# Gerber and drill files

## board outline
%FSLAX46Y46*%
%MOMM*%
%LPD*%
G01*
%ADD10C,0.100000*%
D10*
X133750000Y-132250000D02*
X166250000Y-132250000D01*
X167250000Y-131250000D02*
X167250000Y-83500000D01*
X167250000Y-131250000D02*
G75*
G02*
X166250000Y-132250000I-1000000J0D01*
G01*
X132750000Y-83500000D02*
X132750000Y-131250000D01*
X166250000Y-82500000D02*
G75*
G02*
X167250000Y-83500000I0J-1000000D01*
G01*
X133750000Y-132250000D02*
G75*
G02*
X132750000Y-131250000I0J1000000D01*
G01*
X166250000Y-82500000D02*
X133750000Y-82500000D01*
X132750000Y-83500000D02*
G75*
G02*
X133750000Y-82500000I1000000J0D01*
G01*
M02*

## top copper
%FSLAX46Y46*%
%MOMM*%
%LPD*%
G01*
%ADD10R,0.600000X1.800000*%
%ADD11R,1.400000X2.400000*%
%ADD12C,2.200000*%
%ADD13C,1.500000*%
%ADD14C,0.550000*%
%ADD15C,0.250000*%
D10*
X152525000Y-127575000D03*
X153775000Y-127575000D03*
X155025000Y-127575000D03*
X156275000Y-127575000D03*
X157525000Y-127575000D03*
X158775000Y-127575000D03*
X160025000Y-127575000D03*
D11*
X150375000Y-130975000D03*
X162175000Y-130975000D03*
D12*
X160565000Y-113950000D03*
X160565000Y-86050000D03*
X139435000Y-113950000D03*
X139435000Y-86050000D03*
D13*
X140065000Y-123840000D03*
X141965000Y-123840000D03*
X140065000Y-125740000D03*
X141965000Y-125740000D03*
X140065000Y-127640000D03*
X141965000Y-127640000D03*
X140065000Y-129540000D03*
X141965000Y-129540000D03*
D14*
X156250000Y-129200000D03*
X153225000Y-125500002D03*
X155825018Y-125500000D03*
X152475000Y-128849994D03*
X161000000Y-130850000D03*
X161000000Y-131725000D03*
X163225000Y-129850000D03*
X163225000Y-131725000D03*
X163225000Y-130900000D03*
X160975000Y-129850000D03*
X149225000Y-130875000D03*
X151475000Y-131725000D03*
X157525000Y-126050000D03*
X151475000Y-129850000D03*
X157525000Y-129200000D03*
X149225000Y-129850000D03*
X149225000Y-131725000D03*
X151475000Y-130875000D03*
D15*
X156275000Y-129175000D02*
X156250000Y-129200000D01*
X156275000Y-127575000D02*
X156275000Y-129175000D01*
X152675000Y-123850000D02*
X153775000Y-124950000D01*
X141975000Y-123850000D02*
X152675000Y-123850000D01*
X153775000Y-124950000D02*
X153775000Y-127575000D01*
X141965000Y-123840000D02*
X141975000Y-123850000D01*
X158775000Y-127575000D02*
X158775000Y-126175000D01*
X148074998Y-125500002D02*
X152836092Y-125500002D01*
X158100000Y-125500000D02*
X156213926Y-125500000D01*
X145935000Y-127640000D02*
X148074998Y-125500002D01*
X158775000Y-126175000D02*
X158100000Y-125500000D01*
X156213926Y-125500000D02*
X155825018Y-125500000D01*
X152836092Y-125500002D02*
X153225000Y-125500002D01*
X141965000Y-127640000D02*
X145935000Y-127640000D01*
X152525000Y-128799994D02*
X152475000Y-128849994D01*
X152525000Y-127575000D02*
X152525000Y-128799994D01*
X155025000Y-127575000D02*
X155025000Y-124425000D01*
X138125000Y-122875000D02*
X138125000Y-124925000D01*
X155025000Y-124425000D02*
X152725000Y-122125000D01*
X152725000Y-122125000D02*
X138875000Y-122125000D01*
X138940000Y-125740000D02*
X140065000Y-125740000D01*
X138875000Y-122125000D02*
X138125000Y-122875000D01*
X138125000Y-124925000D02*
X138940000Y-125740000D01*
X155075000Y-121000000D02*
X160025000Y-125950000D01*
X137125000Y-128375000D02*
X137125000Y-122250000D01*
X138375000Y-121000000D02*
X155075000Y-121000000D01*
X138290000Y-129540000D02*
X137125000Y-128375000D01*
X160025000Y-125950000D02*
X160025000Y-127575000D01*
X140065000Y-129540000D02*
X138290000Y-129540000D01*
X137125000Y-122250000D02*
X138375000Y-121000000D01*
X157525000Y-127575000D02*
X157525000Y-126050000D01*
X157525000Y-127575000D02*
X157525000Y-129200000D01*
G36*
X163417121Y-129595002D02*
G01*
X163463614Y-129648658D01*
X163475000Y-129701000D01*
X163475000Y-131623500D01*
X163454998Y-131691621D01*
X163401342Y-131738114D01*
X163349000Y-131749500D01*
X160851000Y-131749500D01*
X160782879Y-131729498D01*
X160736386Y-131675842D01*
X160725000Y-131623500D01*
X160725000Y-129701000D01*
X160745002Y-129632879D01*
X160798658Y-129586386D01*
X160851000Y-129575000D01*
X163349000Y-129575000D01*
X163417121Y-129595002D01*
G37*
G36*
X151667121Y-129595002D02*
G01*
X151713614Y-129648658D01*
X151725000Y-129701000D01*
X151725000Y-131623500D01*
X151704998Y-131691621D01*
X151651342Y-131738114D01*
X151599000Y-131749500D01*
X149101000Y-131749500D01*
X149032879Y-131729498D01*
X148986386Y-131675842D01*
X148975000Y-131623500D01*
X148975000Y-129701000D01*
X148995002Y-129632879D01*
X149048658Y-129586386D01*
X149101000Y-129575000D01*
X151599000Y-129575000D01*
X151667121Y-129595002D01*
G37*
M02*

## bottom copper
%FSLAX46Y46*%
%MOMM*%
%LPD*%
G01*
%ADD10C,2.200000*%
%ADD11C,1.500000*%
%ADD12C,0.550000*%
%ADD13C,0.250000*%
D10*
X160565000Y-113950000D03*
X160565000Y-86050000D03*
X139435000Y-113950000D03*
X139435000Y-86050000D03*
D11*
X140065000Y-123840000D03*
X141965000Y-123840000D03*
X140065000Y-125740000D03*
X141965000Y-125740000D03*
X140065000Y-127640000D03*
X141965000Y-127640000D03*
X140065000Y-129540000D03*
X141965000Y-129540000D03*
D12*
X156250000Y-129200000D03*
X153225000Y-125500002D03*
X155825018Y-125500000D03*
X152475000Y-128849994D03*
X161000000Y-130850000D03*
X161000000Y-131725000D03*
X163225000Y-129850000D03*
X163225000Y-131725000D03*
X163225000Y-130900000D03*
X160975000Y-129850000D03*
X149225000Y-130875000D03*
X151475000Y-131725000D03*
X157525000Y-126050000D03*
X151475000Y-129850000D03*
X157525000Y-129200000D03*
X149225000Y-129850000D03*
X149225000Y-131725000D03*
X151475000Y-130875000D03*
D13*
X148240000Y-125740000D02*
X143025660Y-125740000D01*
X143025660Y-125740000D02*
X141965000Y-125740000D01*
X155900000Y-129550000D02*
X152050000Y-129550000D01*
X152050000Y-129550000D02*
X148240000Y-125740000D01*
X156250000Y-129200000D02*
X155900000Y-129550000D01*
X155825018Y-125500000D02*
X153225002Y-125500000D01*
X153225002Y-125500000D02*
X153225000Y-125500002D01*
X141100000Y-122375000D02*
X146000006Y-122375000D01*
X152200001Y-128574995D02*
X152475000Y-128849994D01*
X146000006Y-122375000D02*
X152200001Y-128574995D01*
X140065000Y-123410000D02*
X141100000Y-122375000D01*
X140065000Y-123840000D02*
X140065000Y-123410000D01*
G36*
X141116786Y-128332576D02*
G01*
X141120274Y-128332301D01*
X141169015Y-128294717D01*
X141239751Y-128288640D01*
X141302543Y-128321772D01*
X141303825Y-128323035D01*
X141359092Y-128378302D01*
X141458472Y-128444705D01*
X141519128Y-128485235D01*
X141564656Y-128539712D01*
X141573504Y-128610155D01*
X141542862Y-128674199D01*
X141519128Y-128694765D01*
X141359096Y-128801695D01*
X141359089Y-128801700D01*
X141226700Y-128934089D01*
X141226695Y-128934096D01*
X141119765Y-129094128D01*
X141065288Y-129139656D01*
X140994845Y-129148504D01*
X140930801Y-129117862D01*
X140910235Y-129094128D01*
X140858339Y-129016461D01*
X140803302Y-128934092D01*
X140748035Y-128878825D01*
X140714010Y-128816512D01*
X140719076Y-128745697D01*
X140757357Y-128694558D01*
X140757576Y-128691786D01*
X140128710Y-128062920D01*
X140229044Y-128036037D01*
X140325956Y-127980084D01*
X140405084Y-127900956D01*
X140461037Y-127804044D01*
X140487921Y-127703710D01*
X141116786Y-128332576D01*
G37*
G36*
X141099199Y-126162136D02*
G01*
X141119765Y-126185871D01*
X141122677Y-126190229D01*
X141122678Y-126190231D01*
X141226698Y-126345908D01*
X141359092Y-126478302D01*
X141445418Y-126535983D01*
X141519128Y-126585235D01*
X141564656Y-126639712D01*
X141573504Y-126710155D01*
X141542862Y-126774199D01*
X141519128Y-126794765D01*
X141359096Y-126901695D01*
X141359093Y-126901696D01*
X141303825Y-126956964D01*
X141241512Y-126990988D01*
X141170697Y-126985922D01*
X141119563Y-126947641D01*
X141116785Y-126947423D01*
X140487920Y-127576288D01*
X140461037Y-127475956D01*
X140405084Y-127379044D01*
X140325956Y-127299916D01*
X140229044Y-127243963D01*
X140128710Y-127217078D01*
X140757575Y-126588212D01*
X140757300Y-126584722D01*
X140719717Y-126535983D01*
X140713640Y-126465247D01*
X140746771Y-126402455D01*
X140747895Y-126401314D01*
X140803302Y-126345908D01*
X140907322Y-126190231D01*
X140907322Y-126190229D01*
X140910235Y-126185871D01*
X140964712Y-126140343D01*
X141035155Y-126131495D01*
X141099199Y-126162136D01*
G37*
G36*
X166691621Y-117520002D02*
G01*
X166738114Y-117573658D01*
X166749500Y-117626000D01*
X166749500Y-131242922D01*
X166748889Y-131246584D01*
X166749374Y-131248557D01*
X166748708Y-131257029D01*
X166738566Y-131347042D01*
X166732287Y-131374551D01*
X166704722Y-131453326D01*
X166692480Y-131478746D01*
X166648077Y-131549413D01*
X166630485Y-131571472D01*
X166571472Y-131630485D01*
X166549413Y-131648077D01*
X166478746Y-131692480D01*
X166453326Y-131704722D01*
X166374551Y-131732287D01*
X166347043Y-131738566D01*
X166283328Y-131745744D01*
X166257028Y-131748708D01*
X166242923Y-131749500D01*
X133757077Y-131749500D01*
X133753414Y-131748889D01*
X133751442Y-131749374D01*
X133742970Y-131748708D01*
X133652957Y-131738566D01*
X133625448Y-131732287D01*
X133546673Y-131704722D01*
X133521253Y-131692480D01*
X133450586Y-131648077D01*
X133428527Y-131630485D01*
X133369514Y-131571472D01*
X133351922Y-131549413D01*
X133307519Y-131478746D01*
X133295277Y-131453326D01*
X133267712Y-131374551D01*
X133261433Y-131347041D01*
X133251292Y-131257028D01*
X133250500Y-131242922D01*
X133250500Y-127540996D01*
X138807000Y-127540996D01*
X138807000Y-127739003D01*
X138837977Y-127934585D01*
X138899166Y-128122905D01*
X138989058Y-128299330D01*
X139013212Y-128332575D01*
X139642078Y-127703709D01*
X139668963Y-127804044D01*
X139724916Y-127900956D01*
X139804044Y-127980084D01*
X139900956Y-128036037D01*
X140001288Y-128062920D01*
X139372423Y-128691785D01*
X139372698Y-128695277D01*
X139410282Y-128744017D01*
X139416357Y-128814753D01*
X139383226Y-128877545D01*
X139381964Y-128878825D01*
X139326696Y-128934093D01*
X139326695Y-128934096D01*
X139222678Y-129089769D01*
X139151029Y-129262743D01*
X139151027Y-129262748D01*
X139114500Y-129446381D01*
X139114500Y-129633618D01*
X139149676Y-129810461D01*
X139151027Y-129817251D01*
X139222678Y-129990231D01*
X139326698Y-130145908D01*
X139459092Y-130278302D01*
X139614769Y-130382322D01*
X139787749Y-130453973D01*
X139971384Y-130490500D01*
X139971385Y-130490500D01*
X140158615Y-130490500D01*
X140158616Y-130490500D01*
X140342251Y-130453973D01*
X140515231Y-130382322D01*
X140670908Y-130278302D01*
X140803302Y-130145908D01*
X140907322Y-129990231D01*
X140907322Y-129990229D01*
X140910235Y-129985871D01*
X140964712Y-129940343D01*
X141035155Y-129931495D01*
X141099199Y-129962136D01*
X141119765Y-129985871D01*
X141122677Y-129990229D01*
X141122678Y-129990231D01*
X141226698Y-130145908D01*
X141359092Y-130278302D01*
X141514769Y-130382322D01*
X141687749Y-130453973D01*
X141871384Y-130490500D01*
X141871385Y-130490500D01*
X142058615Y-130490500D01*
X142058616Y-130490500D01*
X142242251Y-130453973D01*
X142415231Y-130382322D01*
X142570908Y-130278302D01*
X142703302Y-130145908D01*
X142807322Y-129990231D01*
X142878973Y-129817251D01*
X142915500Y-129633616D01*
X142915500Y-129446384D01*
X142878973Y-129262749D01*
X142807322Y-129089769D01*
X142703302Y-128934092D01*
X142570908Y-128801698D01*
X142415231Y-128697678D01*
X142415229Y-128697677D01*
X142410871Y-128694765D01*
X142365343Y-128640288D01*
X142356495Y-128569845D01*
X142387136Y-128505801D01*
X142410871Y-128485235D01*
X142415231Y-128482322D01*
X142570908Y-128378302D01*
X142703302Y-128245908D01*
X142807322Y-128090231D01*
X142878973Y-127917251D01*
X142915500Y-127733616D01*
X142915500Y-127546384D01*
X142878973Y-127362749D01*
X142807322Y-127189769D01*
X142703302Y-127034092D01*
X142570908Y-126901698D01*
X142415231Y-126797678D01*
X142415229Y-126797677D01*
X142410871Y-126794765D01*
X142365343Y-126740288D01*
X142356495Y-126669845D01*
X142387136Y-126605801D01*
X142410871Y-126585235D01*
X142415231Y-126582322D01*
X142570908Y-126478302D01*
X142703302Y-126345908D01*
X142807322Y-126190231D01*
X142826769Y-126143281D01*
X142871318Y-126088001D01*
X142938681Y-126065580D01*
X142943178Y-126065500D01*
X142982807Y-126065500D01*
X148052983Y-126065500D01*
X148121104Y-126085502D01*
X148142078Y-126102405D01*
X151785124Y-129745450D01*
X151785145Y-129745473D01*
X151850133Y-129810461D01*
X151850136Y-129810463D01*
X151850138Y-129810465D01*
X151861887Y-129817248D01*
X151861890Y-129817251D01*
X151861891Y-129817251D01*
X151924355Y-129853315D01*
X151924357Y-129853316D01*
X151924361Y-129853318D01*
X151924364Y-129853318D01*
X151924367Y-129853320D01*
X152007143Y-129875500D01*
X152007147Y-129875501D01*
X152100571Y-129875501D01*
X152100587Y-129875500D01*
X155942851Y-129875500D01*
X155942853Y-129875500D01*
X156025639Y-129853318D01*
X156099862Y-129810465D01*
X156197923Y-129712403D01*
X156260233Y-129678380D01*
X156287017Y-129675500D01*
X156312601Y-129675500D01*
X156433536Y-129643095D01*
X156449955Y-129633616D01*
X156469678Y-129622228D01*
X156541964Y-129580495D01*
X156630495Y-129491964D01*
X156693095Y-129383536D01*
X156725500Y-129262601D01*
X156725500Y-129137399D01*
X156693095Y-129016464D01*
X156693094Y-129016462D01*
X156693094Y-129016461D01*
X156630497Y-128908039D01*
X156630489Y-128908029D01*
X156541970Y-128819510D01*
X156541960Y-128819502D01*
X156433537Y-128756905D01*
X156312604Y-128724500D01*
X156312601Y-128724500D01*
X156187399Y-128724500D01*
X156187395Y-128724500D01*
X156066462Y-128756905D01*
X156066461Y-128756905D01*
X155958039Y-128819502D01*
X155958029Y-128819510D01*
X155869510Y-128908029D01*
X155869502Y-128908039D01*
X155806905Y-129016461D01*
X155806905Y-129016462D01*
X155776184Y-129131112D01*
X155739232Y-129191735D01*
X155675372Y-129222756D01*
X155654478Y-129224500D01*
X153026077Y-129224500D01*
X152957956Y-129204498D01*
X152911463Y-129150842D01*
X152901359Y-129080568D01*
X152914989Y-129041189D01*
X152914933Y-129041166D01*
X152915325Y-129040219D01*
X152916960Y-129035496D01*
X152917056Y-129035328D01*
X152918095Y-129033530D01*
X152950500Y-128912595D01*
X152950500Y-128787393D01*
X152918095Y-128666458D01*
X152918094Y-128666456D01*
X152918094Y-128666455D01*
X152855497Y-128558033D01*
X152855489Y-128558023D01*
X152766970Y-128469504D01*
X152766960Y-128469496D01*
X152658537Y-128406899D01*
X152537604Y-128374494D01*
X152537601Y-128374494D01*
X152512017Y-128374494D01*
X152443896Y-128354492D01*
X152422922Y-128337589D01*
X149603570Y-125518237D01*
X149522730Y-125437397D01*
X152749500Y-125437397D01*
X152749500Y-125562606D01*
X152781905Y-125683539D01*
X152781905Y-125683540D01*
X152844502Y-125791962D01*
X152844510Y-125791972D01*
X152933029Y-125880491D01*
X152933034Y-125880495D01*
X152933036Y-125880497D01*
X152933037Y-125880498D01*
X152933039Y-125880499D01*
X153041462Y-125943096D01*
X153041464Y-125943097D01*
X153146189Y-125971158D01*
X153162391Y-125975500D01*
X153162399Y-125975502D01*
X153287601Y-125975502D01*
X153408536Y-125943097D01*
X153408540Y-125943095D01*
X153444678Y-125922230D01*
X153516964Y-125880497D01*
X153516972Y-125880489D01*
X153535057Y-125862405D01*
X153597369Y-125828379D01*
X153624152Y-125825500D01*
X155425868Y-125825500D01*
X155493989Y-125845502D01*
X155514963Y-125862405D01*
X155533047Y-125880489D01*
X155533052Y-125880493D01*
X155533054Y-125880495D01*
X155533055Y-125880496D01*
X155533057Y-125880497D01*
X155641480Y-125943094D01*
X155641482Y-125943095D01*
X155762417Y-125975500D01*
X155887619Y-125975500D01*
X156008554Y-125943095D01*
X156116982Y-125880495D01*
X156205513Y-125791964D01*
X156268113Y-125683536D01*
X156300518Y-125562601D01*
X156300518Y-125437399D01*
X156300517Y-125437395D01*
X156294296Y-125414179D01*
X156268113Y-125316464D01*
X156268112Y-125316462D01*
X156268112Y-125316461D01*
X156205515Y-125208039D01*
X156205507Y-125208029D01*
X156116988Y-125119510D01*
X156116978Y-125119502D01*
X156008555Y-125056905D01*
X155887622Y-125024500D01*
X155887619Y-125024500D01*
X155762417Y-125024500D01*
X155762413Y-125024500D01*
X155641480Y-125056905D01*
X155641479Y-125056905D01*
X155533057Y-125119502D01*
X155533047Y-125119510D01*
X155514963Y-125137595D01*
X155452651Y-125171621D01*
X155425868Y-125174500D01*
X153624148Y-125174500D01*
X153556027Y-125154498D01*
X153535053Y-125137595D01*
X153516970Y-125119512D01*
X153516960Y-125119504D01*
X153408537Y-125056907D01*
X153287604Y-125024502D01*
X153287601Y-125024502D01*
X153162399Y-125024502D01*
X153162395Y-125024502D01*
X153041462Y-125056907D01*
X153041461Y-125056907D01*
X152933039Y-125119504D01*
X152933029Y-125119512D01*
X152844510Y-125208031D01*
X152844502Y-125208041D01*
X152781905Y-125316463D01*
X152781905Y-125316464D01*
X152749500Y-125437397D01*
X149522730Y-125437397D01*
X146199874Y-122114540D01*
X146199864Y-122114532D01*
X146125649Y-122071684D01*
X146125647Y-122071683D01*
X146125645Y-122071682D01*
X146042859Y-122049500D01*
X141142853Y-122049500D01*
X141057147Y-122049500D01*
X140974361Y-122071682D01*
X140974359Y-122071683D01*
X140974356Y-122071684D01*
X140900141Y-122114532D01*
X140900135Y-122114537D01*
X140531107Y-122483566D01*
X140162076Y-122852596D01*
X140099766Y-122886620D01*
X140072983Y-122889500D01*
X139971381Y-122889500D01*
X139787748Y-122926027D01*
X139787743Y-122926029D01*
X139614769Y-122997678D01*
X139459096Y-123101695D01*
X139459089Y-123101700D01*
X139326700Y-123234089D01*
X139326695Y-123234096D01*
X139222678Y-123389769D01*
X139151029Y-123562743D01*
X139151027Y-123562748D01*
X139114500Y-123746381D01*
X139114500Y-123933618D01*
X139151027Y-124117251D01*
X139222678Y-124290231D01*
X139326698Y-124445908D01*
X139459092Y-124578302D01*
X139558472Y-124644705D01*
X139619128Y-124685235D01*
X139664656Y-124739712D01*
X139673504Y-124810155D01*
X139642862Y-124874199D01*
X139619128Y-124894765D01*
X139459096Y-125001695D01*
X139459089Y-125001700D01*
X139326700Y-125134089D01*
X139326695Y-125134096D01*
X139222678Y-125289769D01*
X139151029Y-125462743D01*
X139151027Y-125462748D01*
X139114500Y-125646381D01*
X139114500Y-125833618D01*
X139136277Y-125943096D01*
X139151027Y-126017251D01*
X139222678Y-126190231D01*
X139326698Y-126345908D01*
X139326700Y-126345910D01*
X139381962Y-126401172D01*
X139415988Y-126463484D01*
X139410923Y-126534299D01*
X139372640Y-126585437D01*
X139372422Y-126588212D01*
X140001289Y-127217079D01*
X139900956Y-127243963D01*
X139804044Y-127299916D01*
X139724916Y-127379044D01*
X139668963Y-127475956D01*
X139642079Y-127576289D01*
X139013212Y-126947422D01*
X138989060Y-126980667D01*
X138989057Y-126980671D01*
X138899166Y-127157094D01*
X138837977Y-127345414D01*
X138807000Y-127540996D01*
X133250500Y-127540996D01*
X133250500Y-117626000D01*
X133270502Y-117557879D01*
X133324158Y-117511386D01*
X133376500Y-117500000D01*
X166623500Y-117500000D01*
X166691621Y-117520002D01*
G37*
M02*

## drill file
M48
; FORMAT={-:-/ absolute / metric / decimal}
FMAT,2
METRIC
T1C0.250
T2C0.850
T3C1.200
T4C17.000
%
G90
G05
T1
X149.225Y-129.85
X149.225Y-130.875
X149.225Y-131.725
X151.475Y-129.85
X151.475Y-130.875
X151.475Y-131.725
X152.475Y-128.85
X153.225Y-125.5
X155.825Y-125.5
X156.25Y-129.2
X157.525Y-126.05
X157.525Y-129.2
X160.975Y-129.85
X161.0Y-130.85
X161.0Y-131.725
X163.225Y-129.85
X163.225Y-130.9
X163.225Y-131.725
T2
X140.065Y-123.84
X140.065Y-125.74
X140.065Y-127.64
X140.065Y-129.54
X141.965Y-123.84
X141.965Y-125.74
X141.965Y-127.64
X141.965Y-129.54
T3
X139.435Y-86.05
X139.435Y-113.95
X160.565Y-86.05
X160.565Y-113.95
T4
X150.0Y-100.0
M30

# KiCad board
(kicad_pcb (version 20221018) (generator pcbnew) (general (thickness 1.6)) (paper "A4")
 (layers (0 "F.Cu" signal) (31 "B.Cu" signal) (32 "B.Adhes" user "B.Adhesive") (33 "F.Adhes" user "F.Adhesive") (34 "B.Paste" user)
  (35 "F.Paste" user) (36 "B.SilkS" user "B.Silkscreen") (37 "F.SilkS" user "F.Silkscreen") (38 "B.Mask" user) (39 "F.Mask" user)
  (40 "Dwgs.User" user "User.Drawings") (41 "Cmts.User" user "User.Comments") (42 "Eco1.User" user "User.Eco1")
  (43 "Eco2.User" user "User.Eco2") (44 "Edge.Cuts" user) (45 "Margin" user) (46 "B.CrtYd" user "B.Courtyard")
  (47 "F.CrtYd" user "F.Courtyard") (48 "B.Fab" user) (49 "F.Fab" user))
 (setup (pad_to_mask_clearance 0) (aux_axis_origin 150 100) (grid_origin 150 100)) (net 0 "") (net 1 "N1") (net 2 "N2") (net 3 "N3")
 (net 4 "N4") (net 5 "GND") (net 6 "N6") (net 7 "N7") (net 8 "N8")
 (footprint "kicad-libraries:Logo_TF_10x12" (layer "F.Cu") (at 149.96 114.89 180)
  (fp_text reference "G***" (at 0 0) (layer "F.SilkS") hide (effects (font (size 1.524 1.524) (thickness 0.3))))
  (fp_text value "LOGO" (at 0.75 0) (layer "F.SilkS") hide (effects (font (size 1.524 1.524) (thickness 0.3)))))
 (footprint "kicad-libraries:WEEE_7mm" (layer "F.Cu") (at 150 87.1 180)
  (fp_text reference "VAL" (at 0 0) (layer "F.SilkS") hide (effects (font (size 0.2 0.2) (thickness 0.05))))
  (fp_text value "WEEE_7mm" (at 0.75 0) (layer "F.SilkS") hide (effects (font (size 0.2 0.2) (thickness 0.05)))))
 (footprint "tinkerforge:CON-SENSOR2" (layer "F.Cu") (at 156.275 132.175)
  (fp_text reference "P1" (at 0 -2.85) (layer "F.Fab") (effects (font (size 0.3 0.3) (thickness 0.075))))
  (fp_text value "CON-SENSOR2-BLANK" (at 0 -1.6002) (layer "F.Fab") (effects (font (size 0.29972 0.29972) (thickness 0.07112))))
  (pad "1" smd rect (at -3.75 -4.6) (size 0.6 1.8) (layers "F.Cu" "F.Paste" "F.Mask") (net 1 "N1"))
  (pad "2" smd rect (at -2.5 -4.6) (size 0.6 1.8) (layers "F.Cu" "F.Paste" "F.Mask") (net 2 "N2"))
  (pad "3" smd rect (at -1.25 -4.6) (size 0.6 1.8) (layers "F.Cu" "F.Paste" "F.Mask") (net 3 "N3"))
  (pad "4" smd rect (at 0 -4.6) (size 0.6 1.8) (layers "F.Cu" "F.Paste" "F.Mask") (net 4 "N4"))
  (pad "5" smd rect (at 1.25 -4.6) (size 0.6 1.8) (layers "F.Cu" "F.Paste" "F.Mask") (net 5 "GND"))
  (pad "6" smd rect (at 2.5 -4.6) (size 0.6 1.8) (layers "F.Cu" "F.Paste" "F.Mask") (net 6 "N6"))
  (pad "7" smd rect (at 3.75 -4.6) (size 0.6 1.8) (layers "F.Cu" "F.Paste" "F.Mask") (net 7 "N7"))
  (pad "EP" smd rect (at -5.9 -1.2) (size 1.4 2.4) (layers "F.Cu" "F.Paste" "F.Mask") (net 5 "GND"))
  (pad "EP" smd rect (at 5.9 -1.2) (size 1.4 2.4) (layers "F.Cu" "F.Paste" "F.Mask") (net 5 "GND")))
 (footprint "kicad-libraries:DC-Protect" (layer "B.Cu") (at 150 100 180)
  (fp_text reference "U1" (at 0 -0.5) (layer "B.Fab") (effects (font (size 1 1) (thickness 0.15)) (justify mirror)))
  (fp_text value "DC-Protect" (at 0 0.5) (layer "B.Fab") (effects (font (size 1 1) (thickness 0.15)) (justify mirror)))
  (pad "" thru_hole circle (at -10.565 -13.95 180) (size 2.2 2.2) (drill 1.2) (layers "*.Cu" "*.Mask"))
  (pad "" thru_hole circle (at -10.565 13.95 180) (size 2.2 2.2) (drill 1.2) (layers "*.Cu" "*.Mask"))
  (pad "" np_thru_hole circle (at 0 0 180) (size 17 17) (drill 17) (layers "*.Cu" "*.Mask"))
  (pad "" thru_hole circle (at 10.565 -13.95 180) (size 2.2 2.2) (drill 1.2) (layers "*.Cu" "*.Mask"))
  (pad "" thru_hole circle (at 10.565 13.95 180) (size 2.2 2.2) (drill 1.2) (layers "*.Cu" "*.Mask"))
  (pad "1" thru_hole circle (at 9.935 -23.84 180) (size 1.5 1.5) (drill 0.85) (layers "*.Cu" "*.Mask") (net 1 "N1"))
  (pad "2" thru_hole circle (at 8.035 -23.84 180) (size 1.5 1.5) (drill 0.85) (layers "*.Cu" "*.Mask") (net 2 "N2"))
  (pad "3" thru_hole circle (at 9.935 -25.74 180) (size 1.5 1.5) (drill 0.85) (layers "*.Cu" "*.Mask") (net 3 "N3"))
  (pad "4" thru_hole circle (at 8.035 -25.74 180) (size 1.5 1.5) (drill 0.85) (layers "*.Cu" "*.Mask") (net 4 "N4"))
  (pad "5" thru_hole circle (at 9.935 -27.64 180) (size 1.5 1.5) (drill 0.85) (layers "*.Cu" "*.Mask") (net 5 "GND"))
  (pad "6" thru_hole circle (at 8.035 -27.64 180) (size 1.5 1.5) (drill 0.85) (layers "*.Cu" "*.Mask") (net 6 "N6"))
  (pad "7" thru_hole circle (at 9.935 -29.54 180) (size 1.5 1.5) (drill 0.85) (layers "*.Cu" "*.Mask") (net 7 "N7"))
  (pad "8" thru_hole circle (at 8.035 -29.54 180) (size 1.5 1.5) (drill 0.85) (layers "*.Cu" "*.Mask") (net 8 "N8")))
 (gr_line (start 133.75 132.25) (end 166.25 132.25) (stroke (width 0.1) (type solid)) (layer "Edge.Cuts"))
 (gr_line (start 167.25 131.25) (end 167.25 83.5) (stroke (width 0.1) (type solid)) (layer "Edge.Cuts"))
 (gr_arc (start 167.25 131.25) (mid 166.957107 131.957107) (end 166.25 132.25) (stroke (width 0.1) (type solid)) (layer "Edge.Cuts"))
 (gr_line (start 132.75 83.5) (end 132.75 131.25) (stroke (width 0.1) (type solid)) (layer "Edge.Cuts"))
 (gr_arc (start 166.25 82.5) (mid 166.957107 82.792893) (end 167.25 83.5) (stroke (width 0.1) (type solid)) (layer "Edge.Cuts"))
 (gr_arc (start 133.75 132.25) (mid 133.042893 131.957107) (end 132.75 131.25) (stroke (width 0.1) (type solid)) (layer "Edge.Cuts"))
 (gr_line (start 166.25 82.5) (end 133.75 82.5) (stroke (width 0.1) (type solid)) (layer "Edge.Cuts"))
 (gr_arc (start 132.75 83.5) (mid 133.042893 82.792893) (end 133.75 82.5) (stroke (width 0.1) (type solid)) (layer "Edge.Cuts"))
 (segment (start 156.275 129.175) (end 156.25 129.2) (width 0.25) (layer "F.Cu") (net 4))
 (segment (start 156.275 127.575) (end 156.275 129.175) (width 0.25) (layer "F.Cu") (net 4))
 (via (at 156.25 129.2) (size 0.55) (drill 0.25) (layers "F.Cu" "B.Cu") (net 4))
 (segment (start 148.24 125.74) (end 143.02566 125.74) (width 0.25) (layer "B.Cu") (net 4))
 (segment (start 143.02566 125.74) (end 141.965 125.74) (width 0.25) (layer "B.Cu") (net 4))
 (segment (start 155.9 129.55) (end 152.05 129.55) (width 0.25) (layer "B.Cu") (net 4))
 (segment (start 152.05 129.55) (end 148.24 125.74) (width 0.25) (layer "B.Cu") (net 4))
 (segment (start 156.25 129.2) (end 155.9 129.55) (width 0.25) (layer "B.Cu") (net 4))
 (segment (start 152.675 123.85) (end 153.775 124.95) (width 0.25) (layer "F.Cu") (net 2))
 (segment (start 141.975 123.85) (end 152.675 123.85) (width 0.25) (layer "F.Cu") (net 2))
 (segment (start 153.775 124.95) (end 153.775 127.575) (width 0.25) (layer "F.Cu") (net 2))
 (segment (start 141.965 123.84) (end 141.975 123.85) (width 0.25) (layer "F.Cu") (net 2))
 (segment (start 158.775 127.575) (end 158.775 126.175) (width 0.25) (layer "F.Cu") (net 6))
 (segment (start 148.074998 125.500002) (end 152.836092 125.500002) (width 0.25) (layer "F.Cu") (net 6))
 (segment (start 158.1 125.5) (end 156.213926 125.5) (width 0.25) (layer "F.Cu") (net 6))
 (segment (start 145.935 127.64) (end 148.074998 125.500002) (width 0.25) (layer "F.Cu") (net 6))
 (segment (start 158.775 126.175) (end 158.1 125.5) (width 0.25) (layer "F.Cu") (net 6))
 (segment (start 156.213926 125.5) (end 155.825018 125.5) (width 0.25) (layer "F.Cu") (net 6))
 (segment (start 152.836092 125.500002) (end 153.225 125.500002) (width 0.25) (layer "F.Cu") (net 6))
 (segment (start 141.965 127.64) (end 145.935 127.64) (width 0.25) (layer "F.Cu") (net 6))
 (via (at 153.225 125.500002) (size 0.55) (drill 0.25) (layers "F.Cu" "B.Cu") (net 6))
 (via (at 155.825018 125.5) (size 0.55) (drill 0.25) (layers "F.Cu" "B.Cu") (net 6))
 (segment (start 155.825018 125.5) (end 153.225002 125.5) (width 0.25) (layer "B.Cu") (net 6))
 (segment (start 153.225002 125.5) (end 153.225 125.500002) (width 0.25) (layer "B.Cu") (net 6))
 (segment (start 152.525 128.799994) (end 152.475 128.849994) (width 0.25) (layer "F.Cu") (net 1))
 (segment (start 152.525 127.575) (end 152.525 128.799994) (width 0.25) (layer "F.Cu") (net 1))
 (via (at 152.475 128.849994) (size 0.55) (drill 0.25) (layers "F.Cu" "B.Cu") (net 1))
 (segment (start 141.1 122.375) (end 146.000006 122.375) (width 0.25) (layer "B.Cu") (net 1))
 (segment (start 152.200001 128.574995) (end 152.475 128.849994) (width 0.25) (layer "B.Cu") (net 1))
 (segment (start 146.000006 122.375) (end 152.200001 128.574995) (width 0.25) (layer "B.Cu") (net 1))
 (segment (start 140.065 123.41) (end 141.1 122.375) (width 0.25) (layer "B.Cu") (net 1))
 (segment (start 140.065 123.84) (end 140.065 123.41) (width 0.25) (layer "B.Cu") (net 1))
 (segment (start 155.025 127.575) (end 155.025 124.425) (width 0.25) (layer "F.Cu") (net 3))
 (segment (start 138.125 122.875) (end 138.125 124.925) (width 0.25) (layer "F.Cu") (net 3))
 (segment (start 155.025 124.425) (end 152.725 122.125) (width 0.25) (layer "F.Cu") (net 3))
 (segment (start 152.725 122.125) (end 138.875 122.125) (width 0.25) (layer "F.Cu") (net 3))
 (segment (start 138.94 125.74) (end 140.065 125.74) (width 0.25) (layer "F.Cu") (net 3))
 (segment (start 138.875 122.125) (end 138.125 122.875) (width 0.25) (layer "F.Cu") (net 3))
 (segment (start 138.125 124.925) (end 138.94 125.74) (width 0.25) (layer "F.Cu") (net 3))
 (segment (start 155.075 121) (end 160.025 125.95) (width 0.25) (layer "F.Cu") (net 7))
 (segment (start 137.125 128.375) (end 137.125 122.25) (width 0.25) (layer "F.Cu") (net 7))
 (segment (start 138.375 121) (end 155.075 121) (width 0.25) (layer "F.Cu") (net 7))
 (segment (start 138.29 129.54) (end 137.125 128.375) (width 0.25) (layer "F.Cu") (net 7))
 (segment (start 160.025 125.95) (end 160.025 127.575) (width 0.25) (layer "F.Cu") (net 7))
 (segment (start 140.065 129.54) (end 138.29 129.54) (width 0.25) (layer "F.Cu") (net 7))
 (segment (start 137.125 122.25) (end 138.375 121) (width 0.25) (layer "F.Cu") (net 7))
 (segment (start 157.525 127.575) (end 157.525 126.05) (width 0.25) (layer "F.Cu") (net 5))
 (segment (start 157.525 127.575) (end 157.525 129.2) (width 0.25) (layer "F.Cu") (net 5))
 (via (at 161 130.85) (size 0.55) (drill 0.25) (layers "F.Cu" "B.Cu") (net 5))
 (via (at 161 131.725) (size 0.55) (drill 0.25) (layers "F.Cu" "B.Cu") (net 5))
 (via (at 163.225 129.85) (size 0.55) (drill 0.25) (layers "F.Cu" "B.Cu") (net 5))
 (via (at 163.225 131.725) (size 0.55) (drill 0.25) (layers "F.Cu" "B.Cu") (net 5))
 (via (at 163.225 130.9) (size 0.55) (drill 0.25) (layers "F.Cu" "B.Cu") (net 5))
 (via (at 160.975 129.85) (size 0.55) (drill 0.25) (layers "F.Cu" "B.Cu") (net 5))
 (via (at 149.225 130.875) (size 0.55) (drill 0.25) (layers "F.Cu" "B.Cu") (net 5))
 (via (at 151.475 131.725) (size 0.55) (drill 0.25) (layers "F.Cu" "B.Cu") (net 5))
 (via (at 157.525 126.05) (size 0.55) (drill 0.25) (layers "F.Cu" "B.Cu") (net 5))
 (via (at 151.475 129.85) (size 0.55) (drill 0.25) (layers "F.Cu" "B.Cu") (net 5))
 (via (at 157.525 129.2) (size 0.55) (drill 0.25) (layers "F.Cu" "B.Cu") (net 5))
 (via (at 149.225 129.85) (size 0.55) (drill 0.25) (layers "F.Cu" "B.Cu") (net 5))
 (via (at 149.225 131.725) (size 0.55) (drill 0.25) (layers "F.Cu" "B.Cu") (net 5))
 (via (at 151.475 130.875) (size 0.55) (drill 0.25) (layers "F.Cu" "B.Cu") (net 5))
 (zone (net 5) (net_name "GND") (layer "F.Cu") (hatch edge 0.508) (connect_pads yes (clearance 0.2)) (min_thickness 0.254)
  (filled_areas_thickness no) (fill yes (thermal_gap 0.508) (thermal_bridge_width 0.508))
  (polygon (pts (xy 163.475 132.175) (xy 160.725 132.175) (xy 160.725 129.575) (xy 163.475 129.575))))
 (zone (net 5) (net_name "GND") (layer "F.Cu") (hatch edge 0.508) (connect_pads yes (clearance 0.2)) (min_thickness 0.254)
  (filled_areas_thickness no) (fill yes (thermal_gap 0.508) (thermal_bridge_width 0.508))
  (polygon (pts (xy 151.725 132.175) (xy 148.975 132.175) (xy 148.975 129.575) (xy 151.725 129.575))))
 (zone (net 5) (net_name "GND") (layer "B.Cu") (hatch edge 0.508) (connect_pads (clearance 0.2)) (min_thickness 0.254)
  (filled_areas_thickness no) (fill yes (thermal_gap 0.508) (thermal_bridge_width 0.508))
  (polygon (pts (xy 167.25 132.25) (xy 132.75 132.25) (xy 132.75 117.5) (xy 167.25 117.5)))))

